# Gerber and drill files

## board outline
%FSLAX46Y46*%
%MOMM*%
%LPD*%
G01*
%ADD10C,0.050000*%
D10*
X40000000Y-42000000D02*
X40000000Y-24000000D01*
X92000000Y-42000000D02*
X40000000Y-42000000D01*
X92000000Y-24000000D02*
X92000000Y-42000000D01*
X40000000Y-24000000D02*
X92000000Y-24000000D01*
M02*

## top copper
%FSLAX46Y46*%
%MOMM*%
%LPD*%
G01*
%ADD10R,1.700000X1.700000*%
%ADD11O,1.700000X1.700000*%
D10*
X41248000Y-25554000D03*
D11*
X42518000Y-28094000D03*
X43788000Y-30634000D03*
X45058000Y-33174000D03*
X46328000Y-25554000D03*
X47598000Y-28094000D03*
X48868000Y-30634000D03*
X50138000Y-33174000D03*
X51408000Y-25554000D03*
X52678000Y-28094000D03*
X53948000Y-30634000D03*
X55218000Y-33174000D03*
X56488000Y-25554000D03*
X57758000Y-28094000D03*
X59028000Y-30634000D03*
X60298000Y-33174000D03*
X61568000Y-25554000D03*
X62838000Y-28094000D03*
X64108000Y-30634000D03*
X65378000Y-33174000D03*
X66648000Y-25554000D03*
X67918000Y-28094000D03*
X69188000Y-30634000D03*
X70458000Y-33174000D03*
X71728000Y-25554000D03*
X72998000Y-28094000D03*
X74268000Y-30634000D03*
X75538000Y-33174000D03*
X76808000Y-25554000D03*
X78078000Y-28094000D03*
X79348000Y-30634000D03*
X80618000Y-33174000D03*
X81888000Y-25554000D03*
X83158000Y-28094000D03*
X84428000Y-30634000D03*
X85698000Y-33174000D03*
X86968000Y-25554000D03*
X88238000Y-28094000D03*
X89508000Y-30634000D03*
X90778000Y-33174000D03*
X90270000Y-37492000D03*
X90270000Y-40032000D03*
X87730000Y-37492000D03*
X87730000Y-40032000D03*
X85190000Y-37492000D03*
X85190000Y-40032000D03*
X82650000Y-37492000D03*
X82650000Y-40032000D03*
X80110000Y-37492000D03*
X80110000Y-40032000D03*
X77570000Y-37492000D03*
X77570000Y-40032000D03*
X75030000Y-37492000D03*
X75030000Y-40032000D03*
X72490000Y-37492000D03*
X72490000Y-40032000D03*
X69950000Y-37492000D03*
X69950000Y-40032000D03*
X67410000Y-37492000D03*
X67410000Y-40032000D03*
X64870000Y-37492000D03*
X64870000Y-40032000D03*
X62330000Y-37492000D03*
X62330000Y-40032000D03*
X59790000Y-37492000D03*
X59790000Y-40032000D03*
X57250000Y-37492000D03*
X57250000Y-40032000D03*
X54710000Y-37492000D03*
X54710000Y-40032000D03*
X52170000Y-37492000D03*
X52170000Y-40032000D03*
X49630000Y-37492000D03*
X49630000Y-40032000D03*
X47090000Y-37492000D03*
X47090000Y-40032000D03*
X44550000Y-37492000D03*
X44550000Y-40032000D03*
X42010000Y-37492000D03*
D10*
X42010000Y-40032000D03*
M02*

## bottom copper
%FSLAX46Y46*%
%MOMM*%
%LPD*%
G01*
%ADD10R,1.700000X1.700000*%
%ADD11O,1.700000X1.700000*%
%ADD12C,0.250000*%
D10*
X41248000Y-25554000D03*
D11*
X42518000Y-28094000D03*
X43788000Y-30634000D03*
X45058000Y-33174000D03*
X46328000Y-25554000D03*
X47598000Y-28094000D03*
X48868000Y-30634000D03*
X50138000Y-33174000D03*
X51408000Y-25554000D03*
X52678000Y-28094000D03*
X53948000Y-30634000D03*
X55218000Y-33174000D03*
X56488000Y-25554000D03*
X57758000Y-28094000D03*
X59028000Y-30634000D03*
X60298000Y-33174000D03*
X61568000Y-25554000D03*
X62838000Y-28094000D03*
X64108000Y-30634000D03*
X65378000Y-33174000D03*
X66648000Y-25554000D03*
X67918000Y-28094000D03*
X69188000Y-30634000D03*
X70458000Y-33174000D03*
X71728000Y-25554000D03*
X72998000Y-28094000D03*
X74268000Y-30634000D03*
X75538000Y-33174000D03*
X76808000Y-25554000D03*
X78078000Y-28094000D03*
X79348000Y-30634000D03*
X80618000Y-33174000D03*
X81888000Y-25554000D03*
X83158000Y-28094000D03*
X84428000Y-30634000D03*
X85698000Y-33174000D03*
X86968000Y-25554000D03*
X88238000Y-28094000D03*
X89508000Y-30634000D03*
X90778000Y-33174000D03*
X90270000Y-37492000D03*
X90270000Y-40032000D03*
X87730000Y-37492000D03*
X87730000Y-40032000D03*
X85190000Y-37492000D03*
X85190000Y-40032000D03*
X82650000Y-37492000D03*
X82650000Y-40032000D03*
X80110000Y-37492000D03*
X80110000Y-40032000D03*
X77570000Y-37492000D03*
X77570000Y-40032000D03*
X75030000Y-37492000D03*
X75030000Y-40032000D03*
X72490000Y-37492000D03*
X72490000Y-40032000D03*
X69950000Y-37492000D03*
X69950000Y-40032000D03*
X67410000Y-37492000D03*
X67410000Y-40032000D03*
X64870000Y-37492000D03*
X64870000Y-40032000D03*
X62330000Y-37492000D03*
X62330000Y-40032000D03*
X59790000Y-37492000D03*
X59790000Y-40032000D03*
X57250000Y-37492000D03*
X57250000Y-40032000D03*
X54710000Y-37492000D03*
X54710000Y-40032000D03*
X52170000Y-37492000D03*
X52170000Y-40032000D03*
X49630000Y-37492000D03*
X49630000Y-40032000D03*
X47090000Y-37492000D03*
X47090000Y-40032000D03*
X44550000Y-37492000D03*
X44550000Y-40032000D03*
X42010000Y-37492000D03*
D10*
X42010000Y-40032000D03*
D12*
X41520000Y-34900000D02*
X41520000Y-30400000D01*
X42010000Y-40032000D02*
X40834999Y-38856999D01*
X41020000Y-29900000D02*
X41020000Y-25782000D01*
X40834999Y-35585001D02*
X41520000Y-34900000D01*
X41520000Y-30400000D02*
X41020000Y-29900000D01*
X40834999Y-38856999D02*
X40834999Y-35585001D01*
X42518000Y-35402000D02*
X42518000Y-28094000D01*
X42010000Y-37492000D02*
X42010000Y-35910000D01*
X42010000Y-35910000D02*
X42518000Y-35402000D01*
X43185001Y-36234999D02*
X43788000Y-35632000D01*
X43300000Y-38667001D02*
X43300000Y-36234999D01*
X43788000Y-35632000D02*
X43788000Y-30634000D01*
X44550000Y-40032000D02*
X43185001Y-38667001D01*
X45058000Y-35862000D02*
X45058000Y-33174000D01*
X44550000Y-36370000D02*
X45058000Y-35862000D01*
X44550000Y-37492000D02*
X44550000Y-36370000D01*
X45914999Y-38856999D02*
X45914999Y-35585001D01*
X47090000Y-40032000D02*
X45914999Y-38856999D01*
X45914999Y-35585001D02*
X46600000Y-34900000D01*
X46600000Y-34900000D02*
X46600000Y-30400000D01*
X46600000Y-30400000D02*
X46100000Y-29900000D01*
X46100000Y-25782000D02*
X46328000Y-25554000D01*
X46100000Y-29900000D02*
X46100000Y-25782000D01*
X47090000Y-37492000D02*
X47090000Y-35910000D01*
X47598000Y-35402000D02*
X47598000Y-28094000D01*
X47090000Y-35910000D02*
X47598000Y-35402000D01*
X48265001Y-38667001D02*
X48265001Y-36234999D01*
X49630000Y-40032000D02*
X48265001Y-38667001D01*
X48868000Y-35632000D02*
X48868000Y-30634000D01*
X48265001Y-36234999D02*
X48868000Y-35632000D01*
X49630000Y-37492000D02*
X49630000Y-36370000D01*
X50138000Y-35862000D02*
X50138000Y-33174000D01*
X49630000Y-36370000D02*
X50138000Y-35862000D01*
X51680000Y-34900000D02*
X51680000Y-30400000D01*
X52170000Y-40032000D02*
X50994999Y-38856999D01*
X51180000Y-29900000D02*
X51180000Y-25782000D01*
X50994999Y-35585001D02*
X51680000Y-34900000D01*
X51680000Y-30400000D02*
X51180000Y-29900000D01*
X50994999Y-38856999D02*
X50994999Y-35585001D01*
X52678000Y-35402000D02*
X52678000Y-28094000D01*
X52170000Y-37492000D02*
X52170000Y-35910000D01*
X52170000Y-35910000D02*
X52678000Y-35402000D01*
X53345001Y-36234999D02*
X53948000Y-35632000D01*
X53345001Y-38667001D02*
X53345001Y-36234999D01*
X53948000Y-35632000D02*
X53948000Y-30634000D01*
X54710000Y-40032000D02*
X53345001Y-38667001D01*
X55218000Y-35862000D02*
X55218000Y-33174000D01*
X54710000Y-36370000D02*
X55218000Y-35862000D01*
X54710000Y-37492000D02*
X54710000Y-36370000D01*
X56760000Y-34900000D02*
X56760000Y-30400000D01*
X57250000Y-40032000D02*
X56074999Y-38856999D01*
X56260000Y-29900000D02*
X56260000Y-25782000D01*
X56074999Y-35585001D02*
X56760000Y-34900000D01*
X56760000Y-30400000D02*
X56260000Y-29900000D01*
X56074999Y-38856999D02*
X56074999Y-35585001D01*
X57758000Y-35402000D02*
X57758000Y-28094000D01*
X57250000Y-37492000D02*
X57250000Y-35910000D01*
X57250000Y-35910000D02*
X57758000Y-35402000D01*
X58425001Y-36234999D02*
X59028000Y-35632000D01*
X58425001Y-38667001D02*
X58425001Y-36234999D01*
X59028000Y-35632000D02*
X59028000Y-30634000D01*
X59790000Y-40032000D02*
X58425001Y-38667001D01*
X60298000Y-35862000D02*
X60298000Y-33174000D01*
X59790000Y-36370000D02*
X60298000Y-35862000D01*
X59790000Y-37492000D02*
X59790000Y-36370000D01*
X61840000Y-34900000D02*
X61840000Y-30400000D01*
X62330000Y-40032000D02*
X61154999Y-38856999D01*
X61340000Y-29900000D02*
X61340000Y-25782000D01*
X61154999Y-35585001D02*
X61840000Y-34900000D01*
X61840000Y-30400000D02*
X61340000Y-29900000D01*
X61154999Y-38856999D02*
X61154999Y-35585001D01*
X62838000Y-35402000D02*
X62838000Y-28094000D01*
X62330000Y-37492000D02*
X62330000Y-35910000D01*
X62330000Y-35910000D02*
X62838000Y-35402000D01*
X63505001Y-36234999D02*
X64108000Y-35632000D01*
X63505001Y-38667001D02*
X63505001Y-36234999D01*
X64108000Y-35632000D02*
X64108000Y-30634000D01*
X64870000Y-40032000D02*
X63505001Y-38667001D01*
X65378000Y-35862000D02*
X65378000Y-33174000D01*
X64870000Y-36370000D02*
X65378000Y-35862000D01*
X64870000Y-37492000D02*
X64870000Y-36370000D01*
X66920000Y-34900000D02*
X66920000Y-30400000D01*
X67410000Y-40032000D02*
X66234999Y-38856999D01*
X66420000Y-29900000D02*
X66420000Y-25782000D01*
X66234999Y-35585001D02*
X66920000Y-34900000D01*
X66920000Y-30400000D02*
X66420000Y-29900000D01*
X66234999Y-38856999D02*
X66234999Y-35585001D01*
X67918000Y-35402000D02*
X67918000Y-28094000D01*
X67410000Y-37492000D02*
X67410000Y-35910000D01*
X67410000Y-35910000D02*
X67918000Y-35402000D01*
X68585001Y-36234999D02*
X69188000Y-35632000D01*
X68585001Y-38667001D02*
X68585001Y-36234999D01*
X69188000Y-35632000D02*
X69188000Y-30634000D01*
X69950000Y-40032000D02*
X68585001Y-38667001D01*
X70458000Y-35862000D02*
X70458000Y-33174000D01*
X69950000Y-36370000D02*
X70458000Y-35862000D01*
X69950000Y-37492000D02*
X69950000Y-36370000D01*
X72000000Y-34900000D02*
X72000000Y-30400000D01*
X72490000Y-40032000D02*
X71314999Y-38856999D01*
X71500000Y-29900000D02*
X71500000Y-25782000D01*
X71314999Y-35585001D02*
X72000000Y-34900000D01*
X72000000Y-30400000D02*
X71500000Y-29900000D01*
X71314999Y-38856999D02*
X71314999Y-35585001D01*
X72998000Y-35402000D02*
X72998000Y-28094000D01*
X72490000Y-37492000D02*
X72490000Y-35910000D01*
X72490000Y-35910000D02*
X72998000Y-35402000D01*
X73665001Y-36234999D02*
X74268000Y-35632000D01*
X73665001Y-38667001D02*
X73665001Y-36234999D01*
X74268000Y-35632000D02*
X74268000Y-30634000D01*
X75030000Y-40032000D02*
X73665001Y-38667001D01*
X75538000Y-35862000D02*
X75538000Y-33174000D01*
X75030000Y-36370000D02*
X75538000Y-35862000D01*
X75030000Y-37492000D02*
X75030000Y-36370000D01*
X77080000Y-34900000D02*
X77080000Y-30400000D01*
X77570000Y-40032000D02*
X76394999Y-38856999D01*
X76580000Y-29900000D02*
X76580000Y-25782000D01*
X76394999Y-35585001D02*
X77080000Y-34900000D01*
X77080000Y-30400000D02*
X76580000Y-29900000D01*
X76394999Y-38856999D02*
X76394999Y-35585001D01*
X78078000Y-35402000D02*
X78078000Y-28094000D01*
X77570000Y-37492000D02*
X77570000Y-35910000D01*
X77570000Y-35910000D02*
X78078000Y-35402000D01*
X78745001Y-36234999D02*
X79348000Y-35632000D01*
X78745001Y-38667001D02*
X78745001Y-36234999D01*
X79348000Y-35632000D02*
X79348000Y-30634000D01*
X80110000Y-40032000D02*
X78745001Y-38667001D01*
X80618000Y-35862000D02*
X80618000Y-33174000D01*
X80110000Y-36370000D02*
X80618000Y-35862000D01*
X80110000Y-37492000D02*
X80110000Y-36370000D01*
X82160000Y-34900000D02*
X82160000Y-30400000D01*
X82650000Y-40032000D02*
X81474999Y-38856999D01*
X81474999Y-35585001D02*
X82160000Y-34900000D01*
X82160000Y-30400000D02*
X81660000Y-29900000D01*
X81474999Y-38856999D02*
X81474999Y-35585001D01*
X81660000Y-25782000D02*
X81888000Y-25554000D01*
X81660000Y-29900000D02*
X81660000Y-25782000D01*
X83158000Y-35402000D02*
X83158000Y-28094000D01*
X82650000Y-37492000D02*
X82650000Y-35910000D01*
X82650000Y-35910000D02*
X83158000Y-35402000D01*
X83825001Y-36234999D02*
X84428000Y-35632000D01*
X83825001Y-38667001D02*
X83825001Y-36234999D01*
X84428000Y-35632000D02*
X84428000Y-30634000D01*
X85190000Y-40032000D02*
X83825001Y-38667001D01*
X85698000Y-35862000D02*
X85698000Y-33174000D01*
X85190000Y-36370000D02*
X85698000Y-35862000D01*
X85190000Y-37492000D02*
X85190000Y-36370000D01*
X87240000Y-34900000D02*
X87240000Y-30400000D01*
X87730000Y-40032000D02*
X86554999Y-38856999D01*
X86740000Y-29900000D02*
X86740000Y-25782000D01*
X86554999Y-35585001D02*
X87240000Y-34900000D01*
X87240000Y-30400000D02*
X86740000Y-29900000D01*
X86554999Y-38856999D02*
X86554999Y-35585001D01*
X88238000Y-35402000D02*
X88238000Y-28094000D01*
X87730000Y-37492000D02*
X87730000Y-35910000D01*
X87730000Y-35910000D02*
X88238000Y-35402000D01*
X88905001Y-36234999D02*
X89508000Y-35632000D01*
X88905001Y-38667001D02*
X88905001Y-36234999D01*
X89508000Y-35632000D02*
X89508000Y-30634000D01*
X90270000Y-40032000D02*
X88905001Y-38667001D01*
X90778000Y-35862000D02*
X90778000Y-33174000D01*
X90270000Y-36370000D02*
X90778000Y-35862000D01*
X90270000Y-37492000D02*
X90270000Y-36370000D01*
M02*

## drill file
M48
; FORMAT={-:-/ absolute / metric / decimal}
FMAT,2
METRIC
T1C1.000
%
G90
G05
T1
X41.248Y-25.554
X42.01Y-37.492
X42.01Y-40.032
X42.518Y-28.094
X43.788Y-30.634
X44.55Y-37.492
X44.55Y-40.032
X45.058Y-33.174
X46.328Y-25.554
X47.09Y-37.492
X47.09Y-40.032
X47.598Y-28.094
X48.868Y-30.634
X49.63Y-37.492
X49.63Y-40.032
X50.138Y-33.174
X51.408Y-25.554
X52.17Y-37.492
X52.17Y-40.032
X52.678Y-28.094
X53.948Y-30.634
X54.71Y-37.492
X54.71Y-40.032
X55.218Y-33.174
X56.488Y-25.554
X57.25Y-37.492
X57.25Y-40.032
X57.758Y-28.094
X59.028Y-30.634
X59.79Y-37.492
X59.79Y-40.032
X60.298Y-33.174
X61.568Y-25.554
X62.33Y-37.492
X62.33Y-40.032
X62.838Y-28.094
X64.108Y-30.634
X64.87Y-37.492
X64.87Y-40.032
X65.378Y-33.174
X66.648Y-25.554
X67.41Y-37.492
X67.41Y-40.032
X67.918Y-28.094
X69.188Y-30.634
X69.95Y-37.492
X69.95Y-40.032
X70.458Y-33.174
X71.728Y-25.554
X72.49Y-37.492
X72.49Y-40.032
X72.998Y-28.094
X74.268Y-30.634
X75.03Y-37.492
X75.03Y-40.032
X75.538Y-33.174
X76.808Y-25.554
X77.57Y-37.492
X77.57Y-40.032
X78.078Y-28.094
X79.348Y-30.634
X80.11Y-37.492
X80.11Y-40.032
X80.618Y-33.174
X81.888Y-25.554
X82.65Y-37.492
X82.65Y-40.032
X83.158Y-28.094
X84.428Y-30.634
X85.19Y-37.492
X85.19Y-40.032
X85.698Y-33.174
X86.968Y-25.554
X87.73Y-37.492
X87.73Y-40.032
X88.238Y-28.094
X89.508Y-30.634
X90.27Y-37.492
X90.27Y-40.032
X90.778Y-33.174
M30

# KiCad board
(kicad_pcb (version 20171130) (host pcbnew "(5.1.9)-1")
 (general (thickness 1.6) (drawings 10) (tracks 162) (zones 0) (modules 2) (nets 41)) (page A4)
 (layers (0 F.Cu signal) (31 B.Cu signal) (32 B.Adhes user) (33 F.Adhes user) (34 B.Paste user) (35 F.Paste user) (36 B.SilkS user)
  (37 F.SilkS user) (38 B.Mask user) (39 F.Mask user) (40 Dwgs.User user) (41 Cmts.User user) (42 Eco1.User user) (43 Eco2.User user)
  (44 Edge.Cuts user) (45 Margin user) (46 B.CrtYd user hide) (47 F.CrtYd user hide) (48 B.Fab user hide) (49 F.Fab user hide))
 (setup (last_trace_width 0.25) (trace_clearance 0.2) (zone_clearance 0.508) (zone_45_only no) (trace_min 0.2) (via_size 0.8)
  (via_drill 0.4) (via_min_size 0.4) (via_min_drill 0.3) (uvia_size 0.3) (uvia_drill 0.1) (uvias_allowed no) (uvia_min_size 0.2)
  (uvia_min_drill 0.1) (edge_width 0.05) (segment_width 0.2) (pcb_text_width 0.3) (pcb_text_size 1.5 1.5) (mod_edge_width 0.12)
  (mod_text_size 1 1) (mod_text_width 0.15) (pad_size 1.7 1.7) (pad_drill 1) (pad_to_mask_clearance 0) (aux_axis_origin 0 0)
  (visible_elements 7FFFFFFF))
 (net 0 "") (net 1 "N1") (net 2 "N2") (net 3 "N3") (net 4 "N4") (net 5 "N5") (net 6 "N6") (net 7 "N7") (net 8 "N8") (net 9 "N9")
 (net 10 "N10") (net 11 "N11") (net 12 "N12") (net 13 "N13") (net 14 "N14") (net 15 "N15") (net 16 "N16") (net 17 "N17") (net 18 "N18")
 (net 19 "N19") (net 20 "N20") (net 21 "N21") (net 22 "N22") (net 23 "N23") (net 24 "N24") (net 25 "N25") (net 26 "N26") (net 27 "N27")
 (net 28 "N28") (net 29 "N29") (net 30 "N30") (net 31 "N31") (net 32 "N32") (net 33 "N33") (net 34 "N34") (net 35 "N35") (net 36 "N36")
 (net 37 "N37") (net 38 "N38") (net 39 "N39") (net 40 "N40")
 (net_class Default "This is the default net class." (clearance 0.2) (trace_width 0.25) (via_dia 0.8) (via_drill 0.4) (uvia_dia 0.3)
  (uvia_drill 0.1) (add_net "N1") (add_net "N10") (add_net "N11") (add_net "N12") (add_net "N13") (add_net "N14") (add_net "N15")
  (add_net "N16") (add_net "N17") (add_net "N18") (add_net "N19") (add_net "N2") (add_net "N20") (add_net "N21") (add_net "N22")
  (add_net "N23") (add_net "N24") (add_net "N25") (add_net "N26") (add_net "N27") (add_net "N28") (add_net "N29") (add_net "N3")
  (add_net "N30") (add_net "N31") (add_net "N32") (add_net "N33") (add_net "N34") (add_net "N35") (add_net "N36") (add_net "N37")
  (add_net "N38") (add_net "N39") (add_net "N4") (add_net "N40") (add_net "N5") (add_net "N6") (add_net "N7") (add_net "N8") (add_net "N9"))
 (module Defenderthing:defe (layer F.Cu) (at 64.108 29.364)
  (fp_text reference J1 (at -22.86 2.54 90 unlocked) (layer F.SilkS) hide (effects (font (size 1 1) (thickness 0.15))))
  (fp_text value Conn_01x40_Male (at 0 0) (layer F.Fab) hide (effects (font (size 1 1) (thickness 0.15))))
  (pad 1 thru_hole rect (at -22.86 -3.81 90) (size 1.7 1.7) (drill 1) (layers *.Cu *.Mask) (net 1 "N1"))
  (pad 2 thru_hole oval (at -21.59 -1.27 90) (size 1.7 1.7) (drill 1) (layers *.Cu *.Mask) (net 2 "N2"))
  (pad 3 thru_hole oval (at -20.32 1.27 90) (size 1.7 1.7) (drill 1) (layers *.Cu *.Mask) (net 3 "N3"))
  (pad 4 thru_hole oval (at -19.05 3.81 90) (size 1.7 1.7) (drill 1) (layers *.Cu *.Mask) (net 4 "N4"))
  (pad 5 thru_hole oval (at -17.78 -3.81 90) (size 1.7 1.7) (drill 1) (layers *.Cu *.Mask) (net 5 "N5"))
  (pad 6 thru_hole oval (at -16.51 -1.27 90) (size 1.7 1.7) (drill 1) (layers *.Cu *.Mask) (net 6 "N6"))
  (pad 7 thru_hole oval (at -15.24 1.27 90) (size 1.7 1.7) (drill 1) (layers *.Cu *.Mask) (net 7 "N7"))
  (pad 8 thru_hole oval (at -13.97 3.81 90) (size 1.7 1.7) (drill 1) (layers *.Cu *.Mask) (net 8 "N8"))
  (pad 9 thru_hole oval (at -12.7 -3.81 90) (size 1.7 1.7) (drill 1) (layers *.Cu *.Mask) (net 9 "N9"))
  (pad 10 thru_hole oval (at -11.43 -1.27 90) (size 1.7 1.7) (drill 1) (layers *.Cu *.Mask) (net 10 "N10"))
  (pad 11 thru_hole oval (at -10.16 1.27 90) (size 1.7 1.7) (drill 1) (layers *.Cu *.Mask) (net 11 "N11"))
  (pad 12 thru_hole oval (at -8.89 3.81 90) (size 1.7 1.7) (drill 1) (layers *.Cu *.Mask) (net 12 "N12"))
  (pad 13 thru_hole oval (at -7.62 -3.81 90) (size 1.7 1.7) (drill 1) (layers *.Cu *.Mask) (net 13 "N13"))
  (pad 14 thru_hole oval (at -6.35 -1.27 90) (size 1.7 1.7) (drill 1) (layers *.Cu *.Mask) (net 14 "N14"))
  (pad 15 thru_hole oval (at -5.08 1.27 90) (size 1.7 1.7) (drill 1) (layers *.Cu *.Mask) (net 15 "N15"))
  (pad 16 thru_hole oval (at -3.81 3.81 90) (size 1.7 1.7) (drill 1) (layers *.Cu *.Mask) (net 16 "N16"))
  (pad 17 thru_hole oval (at -2.54 -3.81 90) (size 1.7 1.7) (drill 1) (layers *.Cu *.Mask) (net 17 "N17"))
  (pad 18 thru_hole oval (at -1.27 -1.27 90) (size 1.7 1.7) (drill 1) (layers *.Cu *.Mask) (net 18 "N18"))
  (pad 19 thru_hole oval (at 0 1.27 90) (size 1.7 1.7) (drill 1) (layers *.Cu *.Mask) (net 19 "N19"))
  (pad 20 thru_hole oval (at 1.27 3.81 90) (size 1.7 1.7) (drill 1) (layers *.Cu *.Mask) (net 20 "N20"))
  (pad 21 thru_hole oval (at 2.54 -3.81 90) (size 1.7 1.7) (drill 1) (layers *.Cu *.Mask) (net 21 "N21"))
  (pad 22 thru_hole oval (at 3.81 -1.27 90) (size 1.7 1.7) (drill 1) (layers *.Cu *.Mask) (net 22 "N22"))
  (pad 23 thru_hole oval (at 5.08 1.27 90) (size 1.7 1.7) (drill 1) (layers *.Cu *.Mask) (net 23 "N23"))
  (pad 24 thru_hole oval (at 6.35 3.81 90) (size 1.7 1.7) (drill 1) (layers *.Cu *.Mask) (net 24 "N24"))
  (pad 25 thru_hole oval (at 7.62 -3.81 90) (size 1.7 1.7) (drill 1) (layers *.Cu *.Mask) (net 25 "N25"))
  (pad 26 thru_hole oval (at 8.89 -1.27 90) (size 1.7 1.7) (drill 1) (layers *.Cu *.Mask) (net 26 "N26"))
  (pad 27 thru_hole oval (at 10.16 1.27 90) (size 1.7 1.7) (drill 1) (layers *.Cu *.Mask) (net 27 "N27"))
  (pad 28 thru_hole oval (at 11.43 3.81 90) (size 1.7 1.7) (drill 1) (layers *.Cu *.Mask) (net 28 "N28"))
  (pad 29 thru_hole oval (at 12.7 -3.81 90) (size 1.7 1.7) (drill 1) (layers *.Cu *.Mask) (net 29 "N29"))
  (pad 30 thru_hole oval (at 13.97 -1.27 90) (size 1.7 1.7) (drill 1) (layers *.Cu *.Mask) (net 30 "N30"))
  (pad 31 thru_hole oval (at 15.24 1.27 90) (size 1.7 1.7) (drill 1) (layers *.Cu *.Mask) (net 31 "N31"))
  (pad 32 thru_hole oval (at 16.51 3.81 90) (size 1.7 1.7) (drill 1) (layers *.Cu *.Mask) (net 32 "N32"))
  (pad 33 thru_hole oval (at 17.78 -3.81 90) (size 1.7 1.7) (drill 1) (layers *.Cu *.Mask) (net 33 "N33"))
  (pad 34 thru_hole oval (at 19.05 -1.27 90) (size 1.7 1.7) (drill 1) (layers *.Cu *.Mask) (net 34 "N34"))
  (pad 35 thru_hole oval (at 20.32 1.27 90) (size 1.7 1.7) (drill 1) (layers *.Cu *.Mask) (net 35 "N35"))
  (pad 36 thru_hole oval (at 21.59 3.81 90) (size 1.7 1.7) (drill 1) (layers *.Cu *.Mask) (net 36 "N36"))
  (pad 37 thru_hole oval (at 22.86 -3.81 90) (size 1.7 1.7) (drill 1) (layers *.Cu *.Mask) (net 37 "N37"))
  (pad 38 thru_hole oval (at 24.13 -1.27 90) (size 1.7 1.7) (drill 1) (layers *.Cu *.Mask) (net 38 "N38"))
  (pad 39 thru_hole oval (at 25.4 1.27 90) (size 1.7 1.7) (drill 1) (layers *.Cu *.Mask) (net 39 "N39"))
  (pad 40 thru_hole oval (at 26.67 3.81 90) (size 1.7 1.7) (drill 1) (layers *.Cu *.Mask) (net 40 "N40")))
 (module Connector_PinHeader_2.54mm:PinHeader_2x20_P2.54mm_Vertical (layer F.Cu) (at 42.01 40.032 90)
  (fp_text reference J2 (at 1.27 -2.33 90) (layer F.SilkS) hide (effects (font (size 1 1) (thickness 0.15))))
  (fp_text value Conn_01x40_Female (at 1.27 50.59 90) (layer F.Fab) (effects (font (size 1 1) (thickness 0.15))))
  (pad 40 thru_hole oval (at 2.54 48.26 90) (size 1.7 1.7) (drill 1) (layers *.Cu *.Mask) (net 40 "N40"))
  (pad 39 thru_hole oval (at 0 48.26 90) (size 1.7 1.7) (drill 1) (layers *.Cu *.Mask) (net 39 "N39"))
  (pad 38 thru_hole oval (at 2.54 45.72 90) (size 1.7 1.7) (drill 1) (layers *.Cu *.Mask) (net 38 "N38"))
  (pad 37 thru_hole oval (at 0 45.72 90) (size 1.7 1.7) (drill 1) (layers *.Cu *.Mask) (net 37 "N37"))
  (pad 36 thru_hole oval (at 2.54 43.18 90) (size 1.7 1.7) (drill 1) (layers *.Cu *.Mask) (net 36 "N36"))
  (pad 35 thru_hole oval (at 0 43.18 90) (size 1.7 1.7) (drill 1) (layers *.Cu *.Mask) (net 35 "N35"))
  (pad 34 thru_hole oval (at 2.54 40.64 90) (size 1.7 1.7) (drill 1) (layers *.Cu *.Mask) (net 34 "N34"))
  (pad 33 thru_hole oval (at 0 40.64 90) (size 1.7 1.7) (drill 1) (layers *.Cu *.Mask) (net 33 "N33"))
  (pad 32 thru_hole oval (at 2.54 38.1 90) (size 1.7 1.7) (drill 1) (layers *.Cu *.Mask) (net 32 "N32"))
  (pad 31 thru_hole oval (at 0 38.1 90) (size 1.7 1.7) (drill 1) (layers *.Cu *.Mask) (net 31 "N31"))
  (pad 30 thru_hole oval (at 2.54 35.56 90) (size 1.7 1.7) (drill 1) (layers *.Cu *.Mask) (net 30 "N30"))
  (pad 29 thru_hole oval (at 0 35.56 90) (size 1.7 1.7) (drill 1) (layers *.Cu *.Mask) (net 29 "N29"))
  (pad 28 thru_hole oval (at 2.54 33.02 90) (size 1.7 1.7) (drill 1) (layers *.Cu *.Mask) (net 28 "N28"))
  (pad 27 thru_hole oval (at 0 33.02 90) (size 1.7 1.7) (drill 1) (layers *.Cu *.Mask) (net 27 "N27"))
  (pad 26 thru_hole oval (at 2.54 30.48 90) (size 1.7 1.7) (drill 1) (layers *.Cu *.Mask) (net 26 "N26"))
  (pad 25 thru_hole oval (at 0 30.48 90) (size 1.7 1.7) (drill 1) (layers *.Cu *.Mask) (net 25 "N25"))
  (pad 24 thru_hole oval (at 2.54 27.94 90) (size 1.7 1.7) (drill 1) (layers *.Cu *.Mask) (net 24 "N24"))
  (pad 23 thru_hole oval (at 0 27.94 90) (size 1.7 1.7) (drill 1) (layers *.Cu *.Mask) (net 23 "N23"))
  (pad 22 thru_hole oval (at 2.54 25.4 90) (size 1.7 1.7) (drill 1) (layers *.Cu *.Mask) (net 22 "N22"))
  (pad 21 thru_hole oval (at 0 25.4 90) (size 1.7 1.7) (drill 1) (layers *.Cu *.Mask) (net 21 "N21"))
  (pad 20 thru_hole oval (at 2.54 22.86 90) (size 1.7 1.7) (drill 1) (layers *.Cu *.Mask) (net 20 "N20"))
  (pad 19 thru_hole oval (at 0 22.86 90) (size 1.7 1.7) (drill 1) (layers *.Cu *.Mask) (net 19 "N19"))
  (pad 18 thru_hole oval (at 2.54 20.32 90) (size 1.7 1.7) (drill 1) (layers *.Cu *.Mask) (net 18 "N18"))
  (pad 17 thru_hole oval (at 0 20.32 90) (size 1.7 1.7) (drill 1) (layers *.Cu *.Mask) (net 17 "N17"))
  (pad 16 thru_hole oval (at 2.54 17.78 90) (size 1.7 1.7) (drill 1) (layers *.Cu *.Mask) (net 16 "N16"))
  (pad 15 thru_hole oval (at 0 17.78 90) (size 1.7 1.7) (drill 1) (layers *.Cu *.Mask) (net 15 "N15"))
  (pad 14 thru_hole oval (at 2.54 15.24 90) (size 1.7 1.7) (drill 1) (layers *.Cu *.Mask) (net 14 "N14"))
  (pad 13 thru_hole oval (at 0 15.24 90) (size 1.7 1.7) (drill 1) (layers *.Cu *.Mask) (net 13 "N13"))
  (pad 12 thru_hole oval (at 2.54 12.7 90) (size 1.7 1.7) (drill 1) (layers *.Cu *.Mask) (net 12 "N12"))
  (pad 11 thru_hole oval (at 0 12.7 90) (size 1.7 1.7) (drill 1) (layers *.Cu *.Mask) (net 11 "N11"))
  (pad 10 thru_hole oval (at 2.54 10.16 90) (size 1.7 1.7) (drill 1) (layers *.Cu *.Mask) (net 10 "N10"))
  (pad 9 thru_hole oval (at 0 10.16 90) (size 1.7 1.7) (drill 1) (layers *.Cu *.Mask) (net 9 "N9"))
  (pad 8 thru_hole oval (at 2.54 7.62 90) (size 1.7 1.7) (drill 1) (layers *.Cu *.Mask) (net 8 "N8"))
  (pad 7 thru_hole oval (at 0 7.62 90) (size 1.7 1.7) (drill 1) (layers *.Cu *.Mask) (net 7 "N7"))
  (pad 6 thru_hole oval (at 2.54 5.08 90) (size 1.7 1.7) (drill 1) (layers *.Cu *.Mask) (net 6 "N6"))
  (pad 5 thru_hole oval (at 0 5.08 90) (size 1.7 1.7) (drill 1) (layers *.Cu *.Mask) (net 5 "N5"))
  (pad 4 thru_hole oval (at 2.54 2.54 90) (size 1.7 1.7) (drill 1) (layers *.Cu *.Mask) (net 4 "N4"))
  (pad 3 thru_hole oval (at 0 2.54 90) (size 1.7 1.7) (drill 1) (layers *.Cu *.Mask) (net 3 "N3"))
  (pad 2 thru_hole oval (at 2.54 0 90) (size 1.7 1.7) (drill 1) (layers *.Cu *.Mask) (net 2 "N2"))
  (pad 1 thru_hole rect (at 0 0 90) (size 1.7 1.7) (drill 1) (layers *.Cu *.Mask) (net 1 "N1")))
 (gr_line (start 40 42) (end 40 24) (layer Edge.Cuts) (width 0.05))
 (gr_line (start 92 42) (end 40 42) (layer Edge.Cuts) (width 0.05))
 (gr_line (start 92 24) (end 92 42) (layer Edge.Cuts) (width 0.05))
 (gr_line (start 40 24) (end 92 24) (layer Edge.Cuts) (width 0.05))
 (segment (start 41.52 34.9) (end 41.52 30.4) (width 0.25) (layer B.Cu) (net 1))
 (segment (start 42.01 40.032) (end 40.834999 38.856999) (width 0.25) (layer B.Cu) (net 1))
 (segment (start 41.02 29.9) (end 41.02 25.782) (width 0.25) (layer B.Cu) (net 1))
 (segment (start 40.834999 35.585001) (end 41.52 34.9) (width 0.25) (layer B.Cu) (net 1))
 (segment (start 41.52 30.4) (end 41.02 29.9) (width 0.25) (layer B.Cu) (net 1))
 (segment (start 40.834999 38.856999) (end 40.834999 35.585001) (width 0.25) (layer B.Cu) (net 1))
 (segment (start 42.518 35.402) (end 42.518 28.094) (width 0.25) (layer B.Cu) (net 2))
 (segment (start 42.01 37.492) (end 42.01 35.91) (width 0.25) (layer B.Cu) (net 2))
 (segment (start 42.01 35.91) (end 42.518 35.402) (width 0.25) (layer B.Cu) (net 2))
 (segment (start 43.185001 36.234999) (end 43.788 35.632) (width 0.25) (layer B.Cu) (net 3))
 (segment (start 43.3 38.667001) (end 43.3 36.234999) (width 0.25) (layer B.Cu) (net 3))
 (segment (start 43.788 35.632) (end 43.788 30.634) (width 0.25) (layer B.Cu) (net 3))
 (segment (start 44.55 40.032) (end 43.185001 38.667001) (width 0.25) (layer B.Cu) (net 3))
 (segment (start 45.058 35.862) (end 45.058 33.174) (width 0.25) (layer B.Cu) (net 4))
 (segment (start 44.55 36.37) (end 45.058 35.862) (width 0.25) (layer B.Cu) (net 4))
 (segment (start 44.55 37.492) (end 44.55 36.37) (width 0.25) (layer B.Cu) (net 4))
 (segment (start 45.914999 38.856999) (end 45.914999 35.585001) (width 0.25) (layer B.Cu) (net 5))
 (segment (start 47.09 40.032) (end 45.914999 38.856999) (width 0.25) (layer B.Cu) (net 5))
 (segment (start 45.914999 35.585001) (end 46.6 34.9) (width 0.25) (layer B.Cu) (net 5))
 (segment (start 46.6 34.9) (end 46.6 30.4) (width 0.25) (layer B.Cu) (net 5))
 (segment (start 46.6 30.4) (end 46.1 29.9) (width 0.25) (layer B.Cu) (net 5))
 (segment (start 46.1 25.782) (end 46.328 25.554) (width 0.25) (layer B.Cu) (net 5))
 (segment (start 46.1 29.9) (end 46.1 25.782) (width 0.25) (layer B.Cu) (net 5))
 (segment (start 47.09 37.492) (end 47.09 35.91) (width 0.25) (layer B.Cu) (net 6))
 (segment (start 47.598 35.402) (end 47.598 28.094) (width 0.25) (layer B.Cu) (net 6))
 (segment (start 47.09 35.91) (end 47.598 35.402) (width 0.25) (layer B.Cu) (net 6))
 (segment (start 48.265001 38.667001) (end 48.265001 36.234999) (width 0.25) (layer B.Cu) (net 7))
 (segment (start 49.63 40.032) (end 48.265001 38.667001) (width 0.25) (layer B.Cu) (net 7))
 (segment (start 48.868 35.632) (end 48.868 30.634) (width 0.25) (layer B.Cu) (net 7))
 (segment (start 48.265001 36.234999) (end 48.868 35.632) (width 0.25) (layer B.Cu) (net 7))
 (segment (start 49.63 37.492) (end 49.63 36.37) (width 0.25) (layer B.Cu) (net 8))
 (segment (start 50.138 35.862) (end 50.138 33.174) (width 0.25) (layer B.Cu) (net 8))
 (segment (start 49.63 36.37) (end 50.138 35.862) (width 0.25) (layer B.Cu) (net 8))
 (segment (start 51.68 34.9) (end 51.68 30.4) (width 0.25) (layer B.Cu) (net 9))
 (segment (start 52.17 40.032) (end 50.994999 38.856999) (width 0.25) (layer B.Cu) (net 9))
 (segment (start 51.18 29.9) (end 51.18 25.782) (width 0.25) (layer B.Cu) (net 9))
 (segment (start 50.994999 35.585001) (end 51.68 34.9) (width 0.25) (layer B.Cu) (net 9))
 (segment (start 51.68 30.4) (end 51.18 29.9) (width 0.25) (layer B.Cu) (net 9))
 (segment (start 50.994999 38.856999) (end 50.994999 35.585001) (width 0.25) (layer B.Cu) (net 9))
 (segment (start 52.678 35.402) (end 52.678 28.094) (width 0.25) (layer B.Cu) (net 10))
 (segment (start 52.17 37.492) (end 52.17 35.91) (width 0.25) (layer B.Cu) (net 10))
 (segment (start 52.17 35.91) (end 52.678 35.402) (width 0.25) (layer B.Cu) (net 10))
 (segment (start 53.345001 36.234999) (end 53.948 35.632) (width 0.25) (layer B.Cu) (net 11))
 (segment (start 53.345001 38.667001) (end 53.345001 36.234999) (width 0.25) (layer B.Cu) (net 11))
 (segment (start 53.948 35.632) (end 53.948 30.634) (width 0.25) (layer B.Cu) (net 11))
 (segment (start 54.71 40.032) (end 53.345001 38.667001) (width 0.25) (layer B.Cu) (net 11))
 (segment (start 55.218 35.862) (end 55.218 33.174) (width 0.25) (layer B.Cu) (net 12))
 (segment (start 54.71 36.37) (end 55.218 35.862) (width 0.25) (layer B.Cu) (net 12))
 (segment (start 54.71 37.492) (end 54.71 36.37) (width 0.25) (layer B.Cu) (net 12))
 (segment (start 56.76 34.9) (end 56.76 30.4) (width 0.25) (layer B.Cu) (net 13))
 (segment (start 57.25 40.032) (end 56.074999 38.856999) (width 0.25) (layer B.Cu) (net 13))
 (segment (start 56.26 29.9) (end 56.26 25.782) (width 0.25) (layer B.Cu) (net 13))
 (segment (start 56.074999 35.585001) (end 56.76 34.9) (width 0.25) (layer B.Cu) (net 13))
 (segment (start 56.76 30.4) (end 56.26 29.9) (width 0.25) (layer B.Cu) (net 13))
 (segment (start 56.074999 38.856999) (end 56.074999 35.585001) (width 0.25) (layer B.Cu) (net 13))
 (segment (start 57.758 35.402) (end 57.758 28.094) (width 0.25) (layer B.Cu) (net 14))
 (segment (start 57.25 37.492) (end 57.25 35.91) (width 0.25) (layer B.Cu) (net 14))
 (segment (start 57.25 35.91) (end 57.758 35.402) (width 0.25) (layer B.Cu) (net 14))
 (segment (start 58.425001 36.234999) (end 59.028 35.632) (width 0.25) (layer B.Cu) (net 15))
 (segment (start 58.425001 38.667001) (end 58.425001 36.234999) (width 0.25) (layer B.Cu) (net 15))
 (segment (start 59.028 35.632) (end 59.028 30.634) (width 0.25) (layer B.Cu) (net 15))
 (segment (start 59.79 40.032) (end 58.425001 38.667001) (width 0.25) (layer B.Cu) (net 15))
 (segment (start 60.298 35.862) (end 60.298 33.174) (width 0.25) (layer B.Cu) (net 16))
 (segment (start 59.79 36.37) (end 60.298 35.862) (width 0.25) (layer B.Cu) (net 16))
 (segment (start 59.79 37.492) (end 59.79 36.37) (width 0.25) (layer B.Cu) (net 16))
 (segment (start 61.84 34.9) (end 61.84 30.4) (width 0.25) (layer B.Cu) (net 17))
 (segment (start 62.33 40.032) (end 61.154999 38.856999) (width 0.25) (layer B.Cu) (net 17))
 (segment (start 61.34 29.9) (end 61.34 25.782) (width 0.25) (layer B.Cu) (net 17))
 (segment (start 61.154999 35.585001) (end 61.84 34.9) (width 0.25) (layer B.Cu) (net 17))
 (segment (start 61.84 30.4) (end 61.34 29.9) (width 0.25) (layer B.Cu) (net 17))
 (segment (start 61.154999 38.856999) (end 61.154999 35.585001) (width 0.25) (layer B.Cu) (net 17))
 (segment (start 62.838 35.402) (end 62.838 28.094) (width 0.25) (layer B.Cu) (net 18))
 (segment (start 62.33 37.492) (end 62.33 35.91) (width 0.25) (layer B.Cu) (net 18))
 (segment (start 62.33 35.91) (end 62.838 35.402) (width 0.25) (layer B.Cu) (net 18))
 (segment (start 63.505001 36.234999) (end 64.108 35.632) (width 0.25) (layer B.Cu) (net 19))
 (segment (start 63.505001 38.667001) (end 63.505001 36.234999) (width 0.25) (layer B.Cu) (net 19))
 (segment (start 64.108 35.632) (end 64.108 30.634) (width 0.25) (layer B.Cu) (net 19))
 (segment (start 64.87 40.032) (end 63.505001 38.667001) (width 0.25) (layer B.Cu) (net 19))
 (segment (start 65.378 35.862) (end 65.378 33.174) (width 0.25) (layer B.Cu) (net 20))
 (segment (start 64.87 36.37) (end 65.378 35.862) (width 0.25) (layer B.Cu) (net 20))
 (segment (start 64.87 37.492) (end 64.87 36.37) (width 0.25) (layer B.Cu) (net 20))
 (segment (start 66.92 34.9) (end 66.92 30.4) (width 0.25) (layer B.Cu) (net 21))
 (segment (start 67.41 40.032) (end 66.234999 38.856999) (width 0.25) (layer B.Cu) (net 21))
 (segment (start 66.42 29.9) (end 66.42 25.782) (width 0.25) (layer B.Cu) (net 21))
 (segment (start 66.234999 35.585001) (end 66.92 34.9) (width 0.25) (layer B.Cu) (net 21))
 (segment (start 66.92 30.4) (end 66.42 29.9) (width 0.25) (layer B.Cu) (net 21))
 (segment (start 66.234999 38.856999) (end 66.234999 35.585001) (width 0.25) (layer B.Cu) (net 21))
 (segment (start 67.918 35.402) (end 67.918 28.094) (width 0.25) (layer B.Cu) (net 22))
 (segment (start 67.41 37.492) (end 67.41 35.91) (width 0.25) (layer B.Cu) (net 22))
 (segment (start 67.41 35.91) (end 67.918 35.402) (width 0.25) (layer B.Cu) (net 22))
 (segment (start 68.585001 36.234999) (end 69.188 35.632) (width 0.25) (layer B.Cu) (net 23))
 (segment (start 68.585001 38.667001) (end 68.585001 36.234999) (width 0.25) (layer B.Cu) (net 23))
 (segment (start 69.188 35.632) (end 69.188 30.634) (width 0.25) (layer B.Cu) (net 23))
 (segment (start 69.95 40.032) (end 68.585001 38.667001) (width 0.25) (layer B.Cu) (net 23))
 (segment (start 70.458 35.862) (end 70.458 33.174) (width 0.25) (layer B.Cu) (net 24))
 (segment (start 69.95 36.37) (end 70.458 35.862) (width 0.25) (layer B.Cu) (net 24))
 (segment (start 69.95 37.492) (end 69.95 36.37) (width 0.25) (layer B.Cu) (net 24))
 (segment (start 72 34.9) (end 72 30.4) (width 0.25) (layer B.Cu) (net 25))
 (segment (start 72.49 40.032) (end 71.314999 38.856999) (width 0.25) (layer B.Cu) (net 25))
 (segment (start 71.5 29.9) (end 71.5 25.782) (width 0.25) (layer B.Cu) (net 25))
 (segment (start 71.314999 35.585001) (end 72 34.9) (width 0.25) (layer B.Cu) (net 25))
 (segment (start 72 30.4) (end 71.5 29.9) (width 0.25) (layer B.Cu) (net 25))
 (segment (start 71.314999 38.856999) (end 71.314999 35.585001) (width 0.25) (layer B.Cu) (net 25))
 (segment (start 72.998 35.402) (end 72.998 28.094) (width 0.25) (layer B.Cu) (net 26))
 (segment (start 72.49 37.492) (end 72.49 35.91) (width 0.25) (layer B.Cu) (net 26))
 (segment (start 72.49 35.91) (end 72.998 35.402) (width 0.25) (layer B.Cu) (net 26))
 (segment (start 73.665001 36.234999) (end 74.268 35.632) (width 0.25) (layer B.Cu) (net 27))
 (segment (start 73.665001 38.667001) (end 73.665001 36.234999) (width 0.25) (layer B.Cu) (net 27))
 (segment (start 74.268 35.632) (end 74.268 30.634) (width 0.25) (layer B.Cu) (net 27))
 (segment (start 75.03 40.032) (end 73.665001 38.667001) (width 0.25) (layer B.Cu) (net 27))
 (segment (start 75.538 35.862) (end 75.538 33.174) (width 0.25) (layer B.Cu) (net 28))
 (segment (start 75.03 36.37) (end 75.538 35.862) (width 0.25) (layer B.Cu) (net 28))
 (segment (start 75.03 37.492) (end 75.03 36.37) (width 0.25) (layer B.Cu) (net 28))
 (segment (start 77.08 34.9) (end 77.08 30.4) (width 0.25) (layer B.Cu) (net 29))
 (segment (start 77.57 40.032) (end 76.394999 38.856999) (width 0.25) (layer B.Cu) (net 29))
 (segment (start 76.58 29.9) (end 76.58 25.782) (width 0.25) (layer B.Cu) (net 29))
 (segment (start 76.394999 35.585001) (end 77.08 34.9) (width 0.25) (layer B.Cu) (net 29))
 (segment (start 77.08 30.4) (end 76.58 29.9) (width 0.25) (layer B.Cu) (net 29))
 (segment (start 76.394999 38.856999) (end 76.394999 35.585001) (width 0.25) (layer B.Cu) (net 29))
 (segment (start 78.078 35.402) (end 78.078 28.094) (width 0.25) (layer B.Cu) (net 30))
 (segment (start 77.57 37.492) (end 77.57 35.91) (width 0.25) (layer B.Cu) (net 30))
 (segment (start 77.57 35.91) (end 78.078 35.402) (width 0.25) (layer B.Cu) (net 30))
 (segment (start 78.745001 36.234999) (end 79.348 35.632) (width 0.25) (layer B.Cu) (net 31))
 (segment (start 78.745001 38.667001) (end 78.745001 36.234999) (width 0.25) (layer B.Cu) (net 31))
 (segment (start 79.348 35.632) (end 79.348 30.634) (width 0.25) (layer B.Cu) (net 31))
 (segment (start 80.11 40.032) (end 78.745001 38.667001) (width 0.25) (layer B.Cu) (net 31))
 (segment (start 80.618 35.862) (end 80.618 33.174) (width 0.25) (layer B.Cu) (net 32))
 (segment (start 80.11 36.37) (end 80.618 35.862) (width 0.25) (layer B.Cu) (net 32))
 (segment (start 80.11 37.492) (end 80.11 36.37) (width 0.25) (layer B.Cu) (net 32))
 (segment (start 82.16 34.9) (end 82.16 30.4) (width 0.25) (layer B.Cu) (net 33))
 (segment (start 82.65 40.032) (end 81.474999 38.856999) (width 0.25) (layer B.Cu) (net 33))
 (segment (start 81.474999 35.585001) (end 82.16 34.9) (width 0.25) (layer B.Cu) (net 33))
 (segment (start 82.16 30.4) (end 81.66 29.9) (width 0.25) (layer B.Cu) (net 33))
 (segment (start 81.474999 38.856999) (end 81.474999 35.585001) (width 0.25) (layer B.Cu) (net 33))
 (segment (start 81.66 25.782) (end 81.888 25.554) (width 0.25) (layer B.Cu) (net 33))
 (segment (start 81.66 29.9) (end 81.66 25.782) (width 0.25) (layer B.Cu) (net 33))
 (segment (start 83.158 35.402) (end 83.158 28.094) (width 0.25) (layer B.Cu) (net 34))
 (segment (start 82.65 37.492) (end 82.65 35.91) (width 0.25) (layer B.Cu) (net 34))
 (segment (start 82.65 35.91) (end 83.158 35.402) (width 0.25) (layer B.Cu) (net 34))
 (segment (start 83.825001 36.234999) (end 84.428 35.632) (width 0.25) (layer B.Cu) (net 35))
 (segment (start 83.825001 38.667001) (end 83.825001 36.234999) (width 0.25) (layer B.Cu) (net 35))
 (segment (start 84.428 35.632) (end 84.428 30.634) (width 0.25) (layer B.Cu) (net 35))
 (segment (start 85.19 40.032) (end 83.825001 38.667001) (width 0.25) (layer B.Cu) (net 35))
 (segment (start 85.698 35.862) (end 85.698 33.174) (width 0.25) (layer B.Cu) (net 36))
 (segment (start 85.19 36.37) (end 85.698 35.862) (width 0.25) (layer B.Cu) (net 36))
 (segment (start 85.19 37.492) (end 85.19 36.37) (width 0.25) (layer B.Cu) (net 36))
 (segment (start 87.24 34.9) (end 87.24 30.4) (width 0.25) (layer B.Cu) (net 37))
 (segment (start 87.73 40.032) (end 86.554999 38.856999) (width 0.25) (layer B.Cu) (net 37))
 (segment (start 86.74 29.9) (end 86.74 25.782) (width 0.25) (layer B.Cu) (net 37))
 (segment (start 86.554999 35.585001) (end 87.24 34.9) (width 0.25) (layer B.Cu) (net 37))
 (segment (start 87.24 30.4) (end 86.74 29.9) (width 0.25) (layer B.Cu) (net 37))
 (segment (start 86.554999 38.856999) (end 86.554999 35.585001) (width 0.25) (layer B.Cu) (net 37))
 (segment (start 88.238 35.402) (end 88.238 28.094) (width 0.25) (layer B.Cu) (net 38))
 (segment (start 87.73 37.492) (end 87.73 35.91) (width 0.25) (layer B.Cu) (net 38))
 (segment (start 87.73 35.91) (end 88.238 35.402) (width 0.25) (layer B.Cu) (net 38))
 (segment (start 88.905001 36.234999) (end 89.508 35.632) (width 0.25) (layer B.Cu) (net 39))
 (segment (start 88.905001 38.667001) (end 88.905001 36.234999) (width 0.25) (layer B.Cu) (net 39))
 (segment (start 89.508 35.632) (end 89.508 30.634) (width 0.25) (layer B.Cu) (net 39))
 (segment (start 90.27 40.032) (end 88.905001 38.667001) (width 0.25) (layer B.Cu) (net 39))
 (segment (start 90.778 35.862) (end 90.778 33.174) (width 0.25) (layer B.Cu) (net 40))
 (segment (start 90.27 36.37) (end 90.778 35.862) (width 0.25) (layer B.Cu) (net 40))
 (segment (start 90.27 37.492) (end 90.27 36.37) (width 0.25) (layer B.Cu) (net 40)))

